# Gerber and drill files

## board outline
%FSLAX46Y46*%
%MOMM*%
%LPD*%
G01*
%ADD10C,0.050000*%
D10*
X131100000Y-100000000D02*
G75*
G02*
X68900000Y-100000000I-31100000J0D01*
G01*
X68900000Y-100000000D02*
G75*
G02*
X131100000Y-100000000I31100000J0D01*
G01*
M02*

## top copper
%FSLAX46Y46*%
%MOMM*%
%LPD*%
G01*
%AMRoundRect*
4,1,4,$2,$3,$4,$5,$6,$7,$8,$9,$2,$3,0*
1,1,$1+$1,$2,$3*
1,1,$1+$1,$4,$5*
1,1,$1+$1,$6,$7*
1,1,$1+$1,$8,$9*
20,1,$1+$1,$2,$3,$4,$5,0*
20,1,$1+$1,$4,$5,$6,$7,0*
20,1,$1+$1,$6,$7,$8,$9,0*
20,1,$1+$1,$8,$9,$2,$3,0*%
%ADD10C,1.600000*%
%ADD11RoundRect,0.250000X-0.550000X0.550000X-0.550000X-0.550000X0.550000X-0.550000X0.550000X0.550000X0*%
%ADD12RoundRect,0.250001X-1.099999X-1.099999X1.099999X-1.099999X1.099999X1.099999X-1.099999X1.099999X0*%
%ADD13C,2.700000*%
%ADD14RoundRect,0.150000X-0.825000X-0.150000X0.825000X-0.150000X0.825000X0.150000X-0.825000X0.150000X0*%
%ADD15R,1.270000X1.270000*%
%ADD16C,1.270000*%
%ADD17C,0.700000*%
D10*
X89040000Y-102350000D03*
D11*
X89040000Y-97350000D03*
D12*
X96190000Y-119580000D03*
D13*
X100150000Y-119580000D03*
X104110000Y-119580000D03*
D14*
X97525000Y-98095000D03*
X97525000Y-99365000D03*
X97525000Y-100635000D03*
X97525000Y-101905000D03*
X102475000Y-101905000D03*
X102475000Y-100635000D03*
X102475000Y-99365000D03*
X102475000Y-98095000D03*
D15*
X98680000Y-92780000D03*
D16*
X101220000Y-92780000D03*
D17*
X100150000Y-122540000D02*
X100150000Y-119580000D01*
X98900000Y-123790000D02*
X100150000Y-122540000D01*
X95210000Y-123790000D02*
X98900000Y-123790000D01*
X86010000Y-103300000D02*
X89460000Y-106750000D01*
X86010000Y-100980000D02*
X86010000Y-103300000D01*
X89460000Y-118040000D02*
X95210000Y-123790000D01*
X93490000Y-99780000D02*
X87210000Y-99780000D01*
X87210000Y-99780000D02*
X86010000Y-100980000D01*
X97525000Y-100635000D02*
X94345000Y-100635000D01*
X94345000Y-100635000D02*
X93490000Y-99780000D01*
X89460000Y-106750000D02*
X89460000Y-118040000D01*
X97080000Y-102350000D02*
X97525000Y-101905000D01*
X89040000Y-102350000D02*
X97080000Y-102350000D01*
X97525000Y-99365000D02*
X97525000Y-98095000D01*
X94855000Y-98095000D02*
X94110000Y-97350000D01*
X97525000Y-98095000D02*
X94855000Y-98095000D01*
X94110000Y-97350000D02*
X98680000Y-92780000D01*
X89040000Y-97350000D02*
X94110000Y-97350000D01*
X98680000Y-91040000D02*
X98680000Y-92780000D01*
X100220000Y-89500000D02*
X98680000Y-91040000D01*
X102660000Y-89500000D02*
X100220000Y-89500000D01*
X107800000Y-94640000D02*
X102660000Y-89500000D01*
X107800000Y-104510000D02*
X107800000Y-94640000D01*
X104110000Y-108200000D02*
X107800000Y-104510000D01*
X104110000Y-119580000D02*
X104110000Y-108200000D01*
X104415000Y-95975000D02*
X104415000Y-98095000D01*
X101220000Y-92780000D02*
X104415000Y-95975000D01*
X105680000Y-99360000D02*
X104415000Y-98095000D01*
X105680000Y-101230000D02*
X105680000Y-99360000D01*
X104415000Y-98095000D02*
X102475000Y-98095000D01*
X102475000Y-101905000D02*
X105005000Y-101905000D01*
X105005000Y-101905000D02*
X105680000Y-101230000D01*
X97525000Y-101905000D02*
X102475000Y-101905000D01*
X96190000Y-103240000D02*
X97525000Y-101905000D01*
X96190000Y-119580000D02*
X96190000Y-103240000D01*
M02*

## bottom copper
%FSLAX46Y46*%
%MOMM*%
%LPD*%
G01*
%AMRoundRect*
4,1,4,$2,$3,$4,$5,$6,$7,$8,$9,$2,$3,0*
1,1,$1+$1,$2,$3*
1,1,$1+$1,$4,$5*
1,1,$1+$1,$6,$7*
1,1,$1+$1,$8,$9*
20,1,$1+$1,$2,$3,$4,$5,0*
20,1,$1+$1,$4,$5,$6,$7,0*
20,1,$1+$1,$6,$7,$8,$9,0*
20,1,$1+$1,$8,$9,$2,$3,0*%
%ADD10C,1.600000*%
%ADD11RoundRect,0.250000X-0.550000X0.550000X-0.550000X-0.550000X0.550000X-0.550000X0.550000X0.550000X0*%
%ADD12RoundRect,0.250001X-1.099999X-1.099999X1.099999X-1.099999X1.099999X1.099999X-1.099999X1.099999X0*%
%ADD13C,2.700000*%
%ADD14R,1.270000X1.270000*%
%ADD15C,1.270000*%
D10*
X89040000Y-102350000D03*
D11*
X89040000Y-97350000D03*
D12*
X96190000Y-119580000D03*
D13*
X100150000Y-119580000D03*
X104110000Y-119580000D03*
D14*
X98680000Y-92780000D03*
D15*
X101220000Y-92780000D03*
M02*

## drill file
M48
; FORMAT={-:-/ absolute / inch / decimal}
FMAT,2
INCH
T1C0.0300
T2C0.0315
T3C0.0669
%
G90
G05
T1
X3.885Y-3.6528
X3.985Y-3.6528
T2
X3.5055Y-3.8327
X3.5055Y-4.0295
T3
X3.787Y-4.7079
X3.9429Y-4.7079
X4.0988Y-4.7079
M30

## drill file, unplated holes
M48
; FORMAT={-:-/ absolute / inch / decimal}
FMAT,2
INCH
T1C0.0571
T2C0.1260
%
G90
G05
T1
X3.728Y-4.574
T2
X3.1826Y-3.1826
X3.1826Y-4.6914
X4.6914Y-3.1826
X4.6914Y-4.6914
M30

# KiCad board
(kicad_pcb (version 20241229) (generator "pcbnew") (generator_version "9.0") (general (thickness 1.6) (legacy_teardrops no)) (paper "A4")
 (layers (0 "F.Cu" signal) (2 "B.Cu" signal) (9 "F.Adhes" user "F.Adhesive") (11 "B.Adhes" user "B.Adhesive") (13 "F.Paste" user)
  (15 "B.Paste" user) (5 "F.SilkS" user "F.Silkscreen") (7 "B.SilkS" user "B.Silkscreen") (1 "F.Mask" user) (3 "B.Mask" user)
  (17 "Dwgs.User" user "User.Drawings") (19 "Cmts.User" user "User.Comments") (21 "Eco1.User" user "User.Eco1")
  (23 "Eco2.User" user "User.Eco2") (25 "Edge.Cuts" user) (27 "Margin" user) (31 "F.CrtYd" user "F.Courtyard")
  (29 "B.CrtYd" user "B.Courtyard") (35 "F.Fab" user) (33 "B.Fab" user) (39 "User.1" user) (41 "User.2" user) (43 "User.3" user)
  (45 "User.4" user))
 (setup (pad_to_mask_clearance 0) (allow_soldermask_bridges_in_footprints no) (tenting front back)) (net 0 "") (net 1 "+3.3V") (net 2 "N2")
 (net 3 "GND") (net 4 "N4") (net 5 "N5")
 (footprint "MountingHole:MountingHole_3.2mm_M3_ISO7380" (layer "F.Cu") (at 80.8374 119.162593)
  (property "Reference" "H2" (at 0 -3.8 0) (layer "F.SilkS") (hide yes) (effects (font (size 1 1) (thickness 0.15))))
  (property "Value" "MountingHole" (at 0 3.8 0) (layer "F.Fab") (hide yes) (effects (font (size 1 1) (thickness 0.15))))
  (pad "" np_thru_hole circle (at 0 0) (size 3.2 3.2) (drill 3.2) (layers "*.Cu" "*.Mask")))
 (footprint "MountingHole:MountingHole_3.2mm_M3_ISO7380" (layer "F.Cu") (at 119.162593 80.8374)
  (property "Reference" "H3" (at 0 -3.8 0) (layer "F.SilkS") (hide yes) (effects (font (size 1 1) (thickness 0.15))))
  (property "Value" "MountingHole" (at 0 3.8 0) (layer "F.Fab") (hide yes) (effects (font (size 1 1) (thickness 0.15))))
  (pad "" np_thru_hole circle (at 0 0) (size 3.2 3.2) (drill 3.2) (layers "*.Cu" "*.Mask")))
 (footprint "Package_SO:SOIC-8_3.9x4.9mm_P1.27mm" (layer "F.Cu") (at 100 100)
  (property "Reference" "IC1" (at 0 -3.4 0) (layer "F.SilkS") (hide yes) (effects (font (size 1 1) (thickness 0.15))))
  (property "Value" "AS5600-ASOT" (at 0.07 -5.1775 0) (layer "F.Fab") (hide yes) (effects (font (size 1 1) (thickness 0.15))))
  (pad "1" smd roundrect (at -2.475 -1.905) (size 1.95 0.6) (layers "F.Cu" "F.Mask" "F.Paste") (roundrect_rratio 0.25) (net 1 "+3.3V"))
  (pad "2" smd roundrect (at -2.475 -0.635) (size 1.95 0.6) (layers "F.Cu" "F.Mask" "F.Paste") (roundrect_rratio 0.25) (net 1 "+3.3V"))
  (pad "3" smd roundrect (at -2.475 0.635) (size 1.95 0.6) (layers "F.Cu" "F.Mask" "F.Paste") (roundrect_rratio 0.25) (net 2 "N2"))
  (pad "4" smd roundrect (at -2.475 1.905) (size 1.95 0.6) (layers "F.Cu" "F.Mask" "F.Paste") (roundrect_rratio 0.25) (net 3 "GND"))
  (pad "5" smd roundrect (at 2.475 1.905) (size 1.95 0.6) (layers "F.Cu" "F.Mask" "F.Paste") (roundrect_rratio 0.25) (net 3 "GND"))
  (pad "6" smd roundrect (at 2.475 0.635) (size 1.95 0.6) (layers "F.Cu" "F.Mask" "F.Paste") (roundrect_rratio 0.25) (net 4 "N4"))
  (pad "7" smd roundrect (at 2.475 -0.635) (size 1.95 0.6) (layers "F.Cu" "F.Mask" "F.Paste") (roundrect_rratio 0.25) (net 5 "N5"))
  (pad "8" smd roundrect (at 2.475 -1.905) (size 1.95 0.6) (layers "F.Cu" "F.Mask" "F.Paste") (roundrect_rratio 0.25) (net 3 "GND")))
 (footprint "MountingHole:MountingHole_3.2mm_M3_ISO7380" (layer "F.Cu") (at 119.162594 119.162594)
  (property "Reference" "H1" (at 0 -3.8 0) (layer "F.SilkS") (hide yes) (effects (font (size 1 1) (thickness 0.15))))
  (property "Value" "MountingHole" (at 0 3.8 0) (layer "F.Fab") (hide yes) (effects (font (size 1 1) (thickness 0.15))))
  (pad "" np_thru_hole circle (at 0 0) (size 3.2 3.2) (drill 3.2) (layers "*.Cu" "*.Mask")))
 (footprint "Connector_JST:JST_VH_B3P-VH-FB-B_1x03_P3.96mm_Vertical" (layer "F.Cu") (at 96.19 119.58)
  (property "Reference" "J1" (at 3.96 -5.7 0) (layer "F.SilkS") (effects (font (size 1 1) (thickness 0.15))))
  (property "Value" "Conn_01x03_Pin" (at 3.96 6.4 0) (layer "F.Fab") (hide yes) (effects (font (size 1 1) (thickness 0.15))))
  (pad "" np_thru_hole circle (at -1.5 -3.4) (size 1.45 1.45) (drill 1.45) (layers "*.Cu" "*.Mask"))
  (pad "1" thru_hole roundrect (at 0 0) (size 2.7 2.7) (drill 1.7) (layers "*.Cu" "*.Mask") (remove_unused_layers no)
   (roundrect_rratio 0.092593) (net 3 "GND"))
  (pad "2" thru_hole circle (at 3.96 0) (size 2.7 2.7) (drill 1.7) (layers "*.Cu" "*.Mask") (remove_unused_layers no) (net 2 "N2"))
  (pad "3" thru_hole circle (at 7.92 0) (size 2.7 2.7) (drill 1.7) (layers "*.Cu" "*.Mask") (remove_unused_layers no) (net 1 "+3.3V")))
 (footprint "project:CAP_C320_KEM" (layer "F.Cu") (at 98.68 92.78)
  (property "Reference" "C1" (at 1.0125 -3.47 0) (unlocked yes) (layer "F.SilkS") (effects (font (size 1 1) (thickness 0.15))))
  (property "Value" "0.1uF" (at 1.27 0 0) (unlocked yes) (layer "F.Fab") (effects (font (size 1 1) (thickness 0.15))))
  (pad "1" thru_hole rect (at 0 0) (size 1.27 1.27) (drill 0.762) (layers "*.Cu" "*.Mask") (remove_unused_layers no) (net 1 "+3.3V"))
  (pad "2" thru_hole circle (at 2.54 0) (size 1.27 1.27) (drill 0.762) (layers "*.Cu" "*.Mask") (remove_unused_layers no) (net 3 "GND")))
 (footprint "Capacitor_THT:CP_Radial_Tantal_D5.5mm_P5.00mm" (layer "F.Cu") (at 89.04 97.35 -90)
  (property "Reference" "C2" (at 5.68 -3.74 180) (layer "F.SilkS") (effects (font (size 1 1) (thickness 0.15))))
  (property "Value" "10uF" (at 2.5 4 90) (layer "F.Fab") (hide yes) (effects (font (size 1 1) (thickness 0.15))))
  (pad "1" thru_hole roundrect (at 0 0 270) (size 1.6 1.6) (drill 0.8) (layers "*.Cu" "*.Mask") (remove_unused_layers no)
   (roundrect_rratio 0.15625) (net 1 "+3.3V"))
  (pad "2" thru_hole circle (at 5 0 270) (size 1.6 1.6) (drill 0.8) (layers "*.Cu" "*.Mask") (remove_unused_layers no) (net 3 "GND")))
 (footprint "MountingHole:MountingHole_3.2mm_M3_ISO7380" (layer "F.Cu") (at 80.8374 80.8374)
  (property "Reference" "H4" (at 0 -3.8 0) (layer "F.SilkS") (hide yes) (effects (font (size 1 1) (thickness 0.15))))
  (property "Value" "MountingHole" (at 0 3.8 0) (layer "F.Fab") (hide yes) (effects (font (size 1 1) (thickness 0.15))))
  (pad "" np_thru_hole circle (at 0 0) (size 3.2 3.2) (drill 3.2) (layers "*.Cu" "*.Mask")))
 (gr_circle (center 100 100) (end 131.1 100) (stroke (width 0.05) (type solid)) (fill no) (layer "Edge.Cuts"))
 (segment (start 102.475 101.905) (end 105.005 101.905) (width 0.7) (layer "F.Cu") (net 3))
 (segment (start 89.04 102.35) (end 97.08 102.35) (width 0.7) (layer "F.Cu") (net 3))
 (segment (start 96.19 103.24) (end 97.525 101.905) (width 0.7) (layer "F.Cu") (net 3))
 (segment (start 105.005 101.905) (end 105.68 101.23) (width 0.7) (layer "F.Cu") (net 3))
 (segment (start 97.08 102.35) (end 97.525 101.905) (width 0.7) (layer "F.Cu") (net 3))
 (segment (start 96.19 119.58) (end 96.19 103.24) (width 0.7) (layer "F.Cu") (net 3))
 (segment (start 97.525 101.905) (end 102.475 101.905) (width 0.7) (layer "F.Cu") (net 3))
 (segment (start 104.415 95.975) (end 104.415 98.095) (width 0.7) (layer "F.Cu") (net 3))
 (segment (start 104.415 98.095) (end 102.475 98.095) (width 0.7) (layer "F.Cu") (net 3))
 (segment (start 101.22 92.78) (end 104.415 95.975) (width 0.7) (layer "F.Cu") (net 3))
 (segment (start 105.68 99.36) (end 104.415 98.095) (width 0.7) (layer "F.Cu") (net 3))
 (segment (start 105.68 101.23) (end 105.68 99.36) (width 0.7) (layer "F.Cu") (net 3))
 (segment (start 102.66 89.5) (end 100.22 89.5) (width 0.7) (layer "F.Cu") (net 1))
 (segment (start 89.04 97.35) (end 94.11 97.35) (width 0.7) (layer "F.Cu") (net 1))
 (segment (start 100.22 89.5) (end 98.68 91.04) (width 0.7) (layer "F.Cu") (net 1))
 (segment (start 97.525 99.365) (end 97.525 98.095) (width 0.7) (layer "F.Cu") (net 1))
 (segment (start 97.525 98.095) (end 94.855 98.095) (width 0.7) (layer "F.Cu") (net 1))
 (segment (start 94.855 98.095) (end 94.11 97.35) (width 0.7) (layer "F.Cu") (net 1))
 (segment (start 107.8 104.51) (end 107.8 94.64) (width 0.7) (layer "F.Cu") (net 1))
 (segment (start 107.8 94.64) (end 102.66 89.5) (width 0.7) (layer "F.Cu") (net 1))
 (segment (start 104.11 108.2) (end 107.8 104.51) (width 0.7) (layer "F.Cu") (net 1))
 (segment (start 94.11 97.35) (end 98.68 92.78) (width 0.7) (layer "F.Cu") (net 1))
 (segment (start 104.11 119.58) (end 104.11 108.2) (width 0.7) (layer "F.Cu") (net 1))
 (segment (start 98.68 91.04) (end 98.68 92.78) (width 0.7) (layer "F.Cu") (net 1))
 (segment (start 97.525 100.635) (end 94.345 100.635) (width 0.7) (layer "F.Cu") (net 2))
 (segment (start 100.15 122.54) (end 100.15 119.58) (width 0.7) (layer "F.Cu") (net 2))
 (segment (start 95.21 123.79) (end 98.9 123.79) (width 0.7) (layer "F.Cu") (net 2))
 (segment (start 93.49 99.78) (end 87.21 99.78) (width 0.7) (layer "F.Cu") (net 2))
 (segment (start 98.9 123.79) (end 100.15 122.54) (width 0.7) (layer "F.Cu") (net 2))
 (segment (start 86.01 103.3) (end 89.46 106.75) (width 0.7) (layer "F.Cu") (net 2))
 (segment (start 87.21 99.78) (end 86.01 100.98) (width 0.7) (layer "F.Cu") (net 2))
 (segment (start 89.46 118.04) (end 95.21 123.79) (width 0.7) (layer "F.Cu") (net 2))
 (segment (start 86.01 100.98) (end 86.01 103.3) (width 0.7) (layer "F.Cu") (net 2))
 (segment (start 94.345 100.635) (end 93.49 99.78) (width 0.7) (layer "F.Cu") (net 2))
 (segment (start 89.46 106.75) (end 89.46 118.04) (width 0.7) (layer "F.Cu") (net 2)))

